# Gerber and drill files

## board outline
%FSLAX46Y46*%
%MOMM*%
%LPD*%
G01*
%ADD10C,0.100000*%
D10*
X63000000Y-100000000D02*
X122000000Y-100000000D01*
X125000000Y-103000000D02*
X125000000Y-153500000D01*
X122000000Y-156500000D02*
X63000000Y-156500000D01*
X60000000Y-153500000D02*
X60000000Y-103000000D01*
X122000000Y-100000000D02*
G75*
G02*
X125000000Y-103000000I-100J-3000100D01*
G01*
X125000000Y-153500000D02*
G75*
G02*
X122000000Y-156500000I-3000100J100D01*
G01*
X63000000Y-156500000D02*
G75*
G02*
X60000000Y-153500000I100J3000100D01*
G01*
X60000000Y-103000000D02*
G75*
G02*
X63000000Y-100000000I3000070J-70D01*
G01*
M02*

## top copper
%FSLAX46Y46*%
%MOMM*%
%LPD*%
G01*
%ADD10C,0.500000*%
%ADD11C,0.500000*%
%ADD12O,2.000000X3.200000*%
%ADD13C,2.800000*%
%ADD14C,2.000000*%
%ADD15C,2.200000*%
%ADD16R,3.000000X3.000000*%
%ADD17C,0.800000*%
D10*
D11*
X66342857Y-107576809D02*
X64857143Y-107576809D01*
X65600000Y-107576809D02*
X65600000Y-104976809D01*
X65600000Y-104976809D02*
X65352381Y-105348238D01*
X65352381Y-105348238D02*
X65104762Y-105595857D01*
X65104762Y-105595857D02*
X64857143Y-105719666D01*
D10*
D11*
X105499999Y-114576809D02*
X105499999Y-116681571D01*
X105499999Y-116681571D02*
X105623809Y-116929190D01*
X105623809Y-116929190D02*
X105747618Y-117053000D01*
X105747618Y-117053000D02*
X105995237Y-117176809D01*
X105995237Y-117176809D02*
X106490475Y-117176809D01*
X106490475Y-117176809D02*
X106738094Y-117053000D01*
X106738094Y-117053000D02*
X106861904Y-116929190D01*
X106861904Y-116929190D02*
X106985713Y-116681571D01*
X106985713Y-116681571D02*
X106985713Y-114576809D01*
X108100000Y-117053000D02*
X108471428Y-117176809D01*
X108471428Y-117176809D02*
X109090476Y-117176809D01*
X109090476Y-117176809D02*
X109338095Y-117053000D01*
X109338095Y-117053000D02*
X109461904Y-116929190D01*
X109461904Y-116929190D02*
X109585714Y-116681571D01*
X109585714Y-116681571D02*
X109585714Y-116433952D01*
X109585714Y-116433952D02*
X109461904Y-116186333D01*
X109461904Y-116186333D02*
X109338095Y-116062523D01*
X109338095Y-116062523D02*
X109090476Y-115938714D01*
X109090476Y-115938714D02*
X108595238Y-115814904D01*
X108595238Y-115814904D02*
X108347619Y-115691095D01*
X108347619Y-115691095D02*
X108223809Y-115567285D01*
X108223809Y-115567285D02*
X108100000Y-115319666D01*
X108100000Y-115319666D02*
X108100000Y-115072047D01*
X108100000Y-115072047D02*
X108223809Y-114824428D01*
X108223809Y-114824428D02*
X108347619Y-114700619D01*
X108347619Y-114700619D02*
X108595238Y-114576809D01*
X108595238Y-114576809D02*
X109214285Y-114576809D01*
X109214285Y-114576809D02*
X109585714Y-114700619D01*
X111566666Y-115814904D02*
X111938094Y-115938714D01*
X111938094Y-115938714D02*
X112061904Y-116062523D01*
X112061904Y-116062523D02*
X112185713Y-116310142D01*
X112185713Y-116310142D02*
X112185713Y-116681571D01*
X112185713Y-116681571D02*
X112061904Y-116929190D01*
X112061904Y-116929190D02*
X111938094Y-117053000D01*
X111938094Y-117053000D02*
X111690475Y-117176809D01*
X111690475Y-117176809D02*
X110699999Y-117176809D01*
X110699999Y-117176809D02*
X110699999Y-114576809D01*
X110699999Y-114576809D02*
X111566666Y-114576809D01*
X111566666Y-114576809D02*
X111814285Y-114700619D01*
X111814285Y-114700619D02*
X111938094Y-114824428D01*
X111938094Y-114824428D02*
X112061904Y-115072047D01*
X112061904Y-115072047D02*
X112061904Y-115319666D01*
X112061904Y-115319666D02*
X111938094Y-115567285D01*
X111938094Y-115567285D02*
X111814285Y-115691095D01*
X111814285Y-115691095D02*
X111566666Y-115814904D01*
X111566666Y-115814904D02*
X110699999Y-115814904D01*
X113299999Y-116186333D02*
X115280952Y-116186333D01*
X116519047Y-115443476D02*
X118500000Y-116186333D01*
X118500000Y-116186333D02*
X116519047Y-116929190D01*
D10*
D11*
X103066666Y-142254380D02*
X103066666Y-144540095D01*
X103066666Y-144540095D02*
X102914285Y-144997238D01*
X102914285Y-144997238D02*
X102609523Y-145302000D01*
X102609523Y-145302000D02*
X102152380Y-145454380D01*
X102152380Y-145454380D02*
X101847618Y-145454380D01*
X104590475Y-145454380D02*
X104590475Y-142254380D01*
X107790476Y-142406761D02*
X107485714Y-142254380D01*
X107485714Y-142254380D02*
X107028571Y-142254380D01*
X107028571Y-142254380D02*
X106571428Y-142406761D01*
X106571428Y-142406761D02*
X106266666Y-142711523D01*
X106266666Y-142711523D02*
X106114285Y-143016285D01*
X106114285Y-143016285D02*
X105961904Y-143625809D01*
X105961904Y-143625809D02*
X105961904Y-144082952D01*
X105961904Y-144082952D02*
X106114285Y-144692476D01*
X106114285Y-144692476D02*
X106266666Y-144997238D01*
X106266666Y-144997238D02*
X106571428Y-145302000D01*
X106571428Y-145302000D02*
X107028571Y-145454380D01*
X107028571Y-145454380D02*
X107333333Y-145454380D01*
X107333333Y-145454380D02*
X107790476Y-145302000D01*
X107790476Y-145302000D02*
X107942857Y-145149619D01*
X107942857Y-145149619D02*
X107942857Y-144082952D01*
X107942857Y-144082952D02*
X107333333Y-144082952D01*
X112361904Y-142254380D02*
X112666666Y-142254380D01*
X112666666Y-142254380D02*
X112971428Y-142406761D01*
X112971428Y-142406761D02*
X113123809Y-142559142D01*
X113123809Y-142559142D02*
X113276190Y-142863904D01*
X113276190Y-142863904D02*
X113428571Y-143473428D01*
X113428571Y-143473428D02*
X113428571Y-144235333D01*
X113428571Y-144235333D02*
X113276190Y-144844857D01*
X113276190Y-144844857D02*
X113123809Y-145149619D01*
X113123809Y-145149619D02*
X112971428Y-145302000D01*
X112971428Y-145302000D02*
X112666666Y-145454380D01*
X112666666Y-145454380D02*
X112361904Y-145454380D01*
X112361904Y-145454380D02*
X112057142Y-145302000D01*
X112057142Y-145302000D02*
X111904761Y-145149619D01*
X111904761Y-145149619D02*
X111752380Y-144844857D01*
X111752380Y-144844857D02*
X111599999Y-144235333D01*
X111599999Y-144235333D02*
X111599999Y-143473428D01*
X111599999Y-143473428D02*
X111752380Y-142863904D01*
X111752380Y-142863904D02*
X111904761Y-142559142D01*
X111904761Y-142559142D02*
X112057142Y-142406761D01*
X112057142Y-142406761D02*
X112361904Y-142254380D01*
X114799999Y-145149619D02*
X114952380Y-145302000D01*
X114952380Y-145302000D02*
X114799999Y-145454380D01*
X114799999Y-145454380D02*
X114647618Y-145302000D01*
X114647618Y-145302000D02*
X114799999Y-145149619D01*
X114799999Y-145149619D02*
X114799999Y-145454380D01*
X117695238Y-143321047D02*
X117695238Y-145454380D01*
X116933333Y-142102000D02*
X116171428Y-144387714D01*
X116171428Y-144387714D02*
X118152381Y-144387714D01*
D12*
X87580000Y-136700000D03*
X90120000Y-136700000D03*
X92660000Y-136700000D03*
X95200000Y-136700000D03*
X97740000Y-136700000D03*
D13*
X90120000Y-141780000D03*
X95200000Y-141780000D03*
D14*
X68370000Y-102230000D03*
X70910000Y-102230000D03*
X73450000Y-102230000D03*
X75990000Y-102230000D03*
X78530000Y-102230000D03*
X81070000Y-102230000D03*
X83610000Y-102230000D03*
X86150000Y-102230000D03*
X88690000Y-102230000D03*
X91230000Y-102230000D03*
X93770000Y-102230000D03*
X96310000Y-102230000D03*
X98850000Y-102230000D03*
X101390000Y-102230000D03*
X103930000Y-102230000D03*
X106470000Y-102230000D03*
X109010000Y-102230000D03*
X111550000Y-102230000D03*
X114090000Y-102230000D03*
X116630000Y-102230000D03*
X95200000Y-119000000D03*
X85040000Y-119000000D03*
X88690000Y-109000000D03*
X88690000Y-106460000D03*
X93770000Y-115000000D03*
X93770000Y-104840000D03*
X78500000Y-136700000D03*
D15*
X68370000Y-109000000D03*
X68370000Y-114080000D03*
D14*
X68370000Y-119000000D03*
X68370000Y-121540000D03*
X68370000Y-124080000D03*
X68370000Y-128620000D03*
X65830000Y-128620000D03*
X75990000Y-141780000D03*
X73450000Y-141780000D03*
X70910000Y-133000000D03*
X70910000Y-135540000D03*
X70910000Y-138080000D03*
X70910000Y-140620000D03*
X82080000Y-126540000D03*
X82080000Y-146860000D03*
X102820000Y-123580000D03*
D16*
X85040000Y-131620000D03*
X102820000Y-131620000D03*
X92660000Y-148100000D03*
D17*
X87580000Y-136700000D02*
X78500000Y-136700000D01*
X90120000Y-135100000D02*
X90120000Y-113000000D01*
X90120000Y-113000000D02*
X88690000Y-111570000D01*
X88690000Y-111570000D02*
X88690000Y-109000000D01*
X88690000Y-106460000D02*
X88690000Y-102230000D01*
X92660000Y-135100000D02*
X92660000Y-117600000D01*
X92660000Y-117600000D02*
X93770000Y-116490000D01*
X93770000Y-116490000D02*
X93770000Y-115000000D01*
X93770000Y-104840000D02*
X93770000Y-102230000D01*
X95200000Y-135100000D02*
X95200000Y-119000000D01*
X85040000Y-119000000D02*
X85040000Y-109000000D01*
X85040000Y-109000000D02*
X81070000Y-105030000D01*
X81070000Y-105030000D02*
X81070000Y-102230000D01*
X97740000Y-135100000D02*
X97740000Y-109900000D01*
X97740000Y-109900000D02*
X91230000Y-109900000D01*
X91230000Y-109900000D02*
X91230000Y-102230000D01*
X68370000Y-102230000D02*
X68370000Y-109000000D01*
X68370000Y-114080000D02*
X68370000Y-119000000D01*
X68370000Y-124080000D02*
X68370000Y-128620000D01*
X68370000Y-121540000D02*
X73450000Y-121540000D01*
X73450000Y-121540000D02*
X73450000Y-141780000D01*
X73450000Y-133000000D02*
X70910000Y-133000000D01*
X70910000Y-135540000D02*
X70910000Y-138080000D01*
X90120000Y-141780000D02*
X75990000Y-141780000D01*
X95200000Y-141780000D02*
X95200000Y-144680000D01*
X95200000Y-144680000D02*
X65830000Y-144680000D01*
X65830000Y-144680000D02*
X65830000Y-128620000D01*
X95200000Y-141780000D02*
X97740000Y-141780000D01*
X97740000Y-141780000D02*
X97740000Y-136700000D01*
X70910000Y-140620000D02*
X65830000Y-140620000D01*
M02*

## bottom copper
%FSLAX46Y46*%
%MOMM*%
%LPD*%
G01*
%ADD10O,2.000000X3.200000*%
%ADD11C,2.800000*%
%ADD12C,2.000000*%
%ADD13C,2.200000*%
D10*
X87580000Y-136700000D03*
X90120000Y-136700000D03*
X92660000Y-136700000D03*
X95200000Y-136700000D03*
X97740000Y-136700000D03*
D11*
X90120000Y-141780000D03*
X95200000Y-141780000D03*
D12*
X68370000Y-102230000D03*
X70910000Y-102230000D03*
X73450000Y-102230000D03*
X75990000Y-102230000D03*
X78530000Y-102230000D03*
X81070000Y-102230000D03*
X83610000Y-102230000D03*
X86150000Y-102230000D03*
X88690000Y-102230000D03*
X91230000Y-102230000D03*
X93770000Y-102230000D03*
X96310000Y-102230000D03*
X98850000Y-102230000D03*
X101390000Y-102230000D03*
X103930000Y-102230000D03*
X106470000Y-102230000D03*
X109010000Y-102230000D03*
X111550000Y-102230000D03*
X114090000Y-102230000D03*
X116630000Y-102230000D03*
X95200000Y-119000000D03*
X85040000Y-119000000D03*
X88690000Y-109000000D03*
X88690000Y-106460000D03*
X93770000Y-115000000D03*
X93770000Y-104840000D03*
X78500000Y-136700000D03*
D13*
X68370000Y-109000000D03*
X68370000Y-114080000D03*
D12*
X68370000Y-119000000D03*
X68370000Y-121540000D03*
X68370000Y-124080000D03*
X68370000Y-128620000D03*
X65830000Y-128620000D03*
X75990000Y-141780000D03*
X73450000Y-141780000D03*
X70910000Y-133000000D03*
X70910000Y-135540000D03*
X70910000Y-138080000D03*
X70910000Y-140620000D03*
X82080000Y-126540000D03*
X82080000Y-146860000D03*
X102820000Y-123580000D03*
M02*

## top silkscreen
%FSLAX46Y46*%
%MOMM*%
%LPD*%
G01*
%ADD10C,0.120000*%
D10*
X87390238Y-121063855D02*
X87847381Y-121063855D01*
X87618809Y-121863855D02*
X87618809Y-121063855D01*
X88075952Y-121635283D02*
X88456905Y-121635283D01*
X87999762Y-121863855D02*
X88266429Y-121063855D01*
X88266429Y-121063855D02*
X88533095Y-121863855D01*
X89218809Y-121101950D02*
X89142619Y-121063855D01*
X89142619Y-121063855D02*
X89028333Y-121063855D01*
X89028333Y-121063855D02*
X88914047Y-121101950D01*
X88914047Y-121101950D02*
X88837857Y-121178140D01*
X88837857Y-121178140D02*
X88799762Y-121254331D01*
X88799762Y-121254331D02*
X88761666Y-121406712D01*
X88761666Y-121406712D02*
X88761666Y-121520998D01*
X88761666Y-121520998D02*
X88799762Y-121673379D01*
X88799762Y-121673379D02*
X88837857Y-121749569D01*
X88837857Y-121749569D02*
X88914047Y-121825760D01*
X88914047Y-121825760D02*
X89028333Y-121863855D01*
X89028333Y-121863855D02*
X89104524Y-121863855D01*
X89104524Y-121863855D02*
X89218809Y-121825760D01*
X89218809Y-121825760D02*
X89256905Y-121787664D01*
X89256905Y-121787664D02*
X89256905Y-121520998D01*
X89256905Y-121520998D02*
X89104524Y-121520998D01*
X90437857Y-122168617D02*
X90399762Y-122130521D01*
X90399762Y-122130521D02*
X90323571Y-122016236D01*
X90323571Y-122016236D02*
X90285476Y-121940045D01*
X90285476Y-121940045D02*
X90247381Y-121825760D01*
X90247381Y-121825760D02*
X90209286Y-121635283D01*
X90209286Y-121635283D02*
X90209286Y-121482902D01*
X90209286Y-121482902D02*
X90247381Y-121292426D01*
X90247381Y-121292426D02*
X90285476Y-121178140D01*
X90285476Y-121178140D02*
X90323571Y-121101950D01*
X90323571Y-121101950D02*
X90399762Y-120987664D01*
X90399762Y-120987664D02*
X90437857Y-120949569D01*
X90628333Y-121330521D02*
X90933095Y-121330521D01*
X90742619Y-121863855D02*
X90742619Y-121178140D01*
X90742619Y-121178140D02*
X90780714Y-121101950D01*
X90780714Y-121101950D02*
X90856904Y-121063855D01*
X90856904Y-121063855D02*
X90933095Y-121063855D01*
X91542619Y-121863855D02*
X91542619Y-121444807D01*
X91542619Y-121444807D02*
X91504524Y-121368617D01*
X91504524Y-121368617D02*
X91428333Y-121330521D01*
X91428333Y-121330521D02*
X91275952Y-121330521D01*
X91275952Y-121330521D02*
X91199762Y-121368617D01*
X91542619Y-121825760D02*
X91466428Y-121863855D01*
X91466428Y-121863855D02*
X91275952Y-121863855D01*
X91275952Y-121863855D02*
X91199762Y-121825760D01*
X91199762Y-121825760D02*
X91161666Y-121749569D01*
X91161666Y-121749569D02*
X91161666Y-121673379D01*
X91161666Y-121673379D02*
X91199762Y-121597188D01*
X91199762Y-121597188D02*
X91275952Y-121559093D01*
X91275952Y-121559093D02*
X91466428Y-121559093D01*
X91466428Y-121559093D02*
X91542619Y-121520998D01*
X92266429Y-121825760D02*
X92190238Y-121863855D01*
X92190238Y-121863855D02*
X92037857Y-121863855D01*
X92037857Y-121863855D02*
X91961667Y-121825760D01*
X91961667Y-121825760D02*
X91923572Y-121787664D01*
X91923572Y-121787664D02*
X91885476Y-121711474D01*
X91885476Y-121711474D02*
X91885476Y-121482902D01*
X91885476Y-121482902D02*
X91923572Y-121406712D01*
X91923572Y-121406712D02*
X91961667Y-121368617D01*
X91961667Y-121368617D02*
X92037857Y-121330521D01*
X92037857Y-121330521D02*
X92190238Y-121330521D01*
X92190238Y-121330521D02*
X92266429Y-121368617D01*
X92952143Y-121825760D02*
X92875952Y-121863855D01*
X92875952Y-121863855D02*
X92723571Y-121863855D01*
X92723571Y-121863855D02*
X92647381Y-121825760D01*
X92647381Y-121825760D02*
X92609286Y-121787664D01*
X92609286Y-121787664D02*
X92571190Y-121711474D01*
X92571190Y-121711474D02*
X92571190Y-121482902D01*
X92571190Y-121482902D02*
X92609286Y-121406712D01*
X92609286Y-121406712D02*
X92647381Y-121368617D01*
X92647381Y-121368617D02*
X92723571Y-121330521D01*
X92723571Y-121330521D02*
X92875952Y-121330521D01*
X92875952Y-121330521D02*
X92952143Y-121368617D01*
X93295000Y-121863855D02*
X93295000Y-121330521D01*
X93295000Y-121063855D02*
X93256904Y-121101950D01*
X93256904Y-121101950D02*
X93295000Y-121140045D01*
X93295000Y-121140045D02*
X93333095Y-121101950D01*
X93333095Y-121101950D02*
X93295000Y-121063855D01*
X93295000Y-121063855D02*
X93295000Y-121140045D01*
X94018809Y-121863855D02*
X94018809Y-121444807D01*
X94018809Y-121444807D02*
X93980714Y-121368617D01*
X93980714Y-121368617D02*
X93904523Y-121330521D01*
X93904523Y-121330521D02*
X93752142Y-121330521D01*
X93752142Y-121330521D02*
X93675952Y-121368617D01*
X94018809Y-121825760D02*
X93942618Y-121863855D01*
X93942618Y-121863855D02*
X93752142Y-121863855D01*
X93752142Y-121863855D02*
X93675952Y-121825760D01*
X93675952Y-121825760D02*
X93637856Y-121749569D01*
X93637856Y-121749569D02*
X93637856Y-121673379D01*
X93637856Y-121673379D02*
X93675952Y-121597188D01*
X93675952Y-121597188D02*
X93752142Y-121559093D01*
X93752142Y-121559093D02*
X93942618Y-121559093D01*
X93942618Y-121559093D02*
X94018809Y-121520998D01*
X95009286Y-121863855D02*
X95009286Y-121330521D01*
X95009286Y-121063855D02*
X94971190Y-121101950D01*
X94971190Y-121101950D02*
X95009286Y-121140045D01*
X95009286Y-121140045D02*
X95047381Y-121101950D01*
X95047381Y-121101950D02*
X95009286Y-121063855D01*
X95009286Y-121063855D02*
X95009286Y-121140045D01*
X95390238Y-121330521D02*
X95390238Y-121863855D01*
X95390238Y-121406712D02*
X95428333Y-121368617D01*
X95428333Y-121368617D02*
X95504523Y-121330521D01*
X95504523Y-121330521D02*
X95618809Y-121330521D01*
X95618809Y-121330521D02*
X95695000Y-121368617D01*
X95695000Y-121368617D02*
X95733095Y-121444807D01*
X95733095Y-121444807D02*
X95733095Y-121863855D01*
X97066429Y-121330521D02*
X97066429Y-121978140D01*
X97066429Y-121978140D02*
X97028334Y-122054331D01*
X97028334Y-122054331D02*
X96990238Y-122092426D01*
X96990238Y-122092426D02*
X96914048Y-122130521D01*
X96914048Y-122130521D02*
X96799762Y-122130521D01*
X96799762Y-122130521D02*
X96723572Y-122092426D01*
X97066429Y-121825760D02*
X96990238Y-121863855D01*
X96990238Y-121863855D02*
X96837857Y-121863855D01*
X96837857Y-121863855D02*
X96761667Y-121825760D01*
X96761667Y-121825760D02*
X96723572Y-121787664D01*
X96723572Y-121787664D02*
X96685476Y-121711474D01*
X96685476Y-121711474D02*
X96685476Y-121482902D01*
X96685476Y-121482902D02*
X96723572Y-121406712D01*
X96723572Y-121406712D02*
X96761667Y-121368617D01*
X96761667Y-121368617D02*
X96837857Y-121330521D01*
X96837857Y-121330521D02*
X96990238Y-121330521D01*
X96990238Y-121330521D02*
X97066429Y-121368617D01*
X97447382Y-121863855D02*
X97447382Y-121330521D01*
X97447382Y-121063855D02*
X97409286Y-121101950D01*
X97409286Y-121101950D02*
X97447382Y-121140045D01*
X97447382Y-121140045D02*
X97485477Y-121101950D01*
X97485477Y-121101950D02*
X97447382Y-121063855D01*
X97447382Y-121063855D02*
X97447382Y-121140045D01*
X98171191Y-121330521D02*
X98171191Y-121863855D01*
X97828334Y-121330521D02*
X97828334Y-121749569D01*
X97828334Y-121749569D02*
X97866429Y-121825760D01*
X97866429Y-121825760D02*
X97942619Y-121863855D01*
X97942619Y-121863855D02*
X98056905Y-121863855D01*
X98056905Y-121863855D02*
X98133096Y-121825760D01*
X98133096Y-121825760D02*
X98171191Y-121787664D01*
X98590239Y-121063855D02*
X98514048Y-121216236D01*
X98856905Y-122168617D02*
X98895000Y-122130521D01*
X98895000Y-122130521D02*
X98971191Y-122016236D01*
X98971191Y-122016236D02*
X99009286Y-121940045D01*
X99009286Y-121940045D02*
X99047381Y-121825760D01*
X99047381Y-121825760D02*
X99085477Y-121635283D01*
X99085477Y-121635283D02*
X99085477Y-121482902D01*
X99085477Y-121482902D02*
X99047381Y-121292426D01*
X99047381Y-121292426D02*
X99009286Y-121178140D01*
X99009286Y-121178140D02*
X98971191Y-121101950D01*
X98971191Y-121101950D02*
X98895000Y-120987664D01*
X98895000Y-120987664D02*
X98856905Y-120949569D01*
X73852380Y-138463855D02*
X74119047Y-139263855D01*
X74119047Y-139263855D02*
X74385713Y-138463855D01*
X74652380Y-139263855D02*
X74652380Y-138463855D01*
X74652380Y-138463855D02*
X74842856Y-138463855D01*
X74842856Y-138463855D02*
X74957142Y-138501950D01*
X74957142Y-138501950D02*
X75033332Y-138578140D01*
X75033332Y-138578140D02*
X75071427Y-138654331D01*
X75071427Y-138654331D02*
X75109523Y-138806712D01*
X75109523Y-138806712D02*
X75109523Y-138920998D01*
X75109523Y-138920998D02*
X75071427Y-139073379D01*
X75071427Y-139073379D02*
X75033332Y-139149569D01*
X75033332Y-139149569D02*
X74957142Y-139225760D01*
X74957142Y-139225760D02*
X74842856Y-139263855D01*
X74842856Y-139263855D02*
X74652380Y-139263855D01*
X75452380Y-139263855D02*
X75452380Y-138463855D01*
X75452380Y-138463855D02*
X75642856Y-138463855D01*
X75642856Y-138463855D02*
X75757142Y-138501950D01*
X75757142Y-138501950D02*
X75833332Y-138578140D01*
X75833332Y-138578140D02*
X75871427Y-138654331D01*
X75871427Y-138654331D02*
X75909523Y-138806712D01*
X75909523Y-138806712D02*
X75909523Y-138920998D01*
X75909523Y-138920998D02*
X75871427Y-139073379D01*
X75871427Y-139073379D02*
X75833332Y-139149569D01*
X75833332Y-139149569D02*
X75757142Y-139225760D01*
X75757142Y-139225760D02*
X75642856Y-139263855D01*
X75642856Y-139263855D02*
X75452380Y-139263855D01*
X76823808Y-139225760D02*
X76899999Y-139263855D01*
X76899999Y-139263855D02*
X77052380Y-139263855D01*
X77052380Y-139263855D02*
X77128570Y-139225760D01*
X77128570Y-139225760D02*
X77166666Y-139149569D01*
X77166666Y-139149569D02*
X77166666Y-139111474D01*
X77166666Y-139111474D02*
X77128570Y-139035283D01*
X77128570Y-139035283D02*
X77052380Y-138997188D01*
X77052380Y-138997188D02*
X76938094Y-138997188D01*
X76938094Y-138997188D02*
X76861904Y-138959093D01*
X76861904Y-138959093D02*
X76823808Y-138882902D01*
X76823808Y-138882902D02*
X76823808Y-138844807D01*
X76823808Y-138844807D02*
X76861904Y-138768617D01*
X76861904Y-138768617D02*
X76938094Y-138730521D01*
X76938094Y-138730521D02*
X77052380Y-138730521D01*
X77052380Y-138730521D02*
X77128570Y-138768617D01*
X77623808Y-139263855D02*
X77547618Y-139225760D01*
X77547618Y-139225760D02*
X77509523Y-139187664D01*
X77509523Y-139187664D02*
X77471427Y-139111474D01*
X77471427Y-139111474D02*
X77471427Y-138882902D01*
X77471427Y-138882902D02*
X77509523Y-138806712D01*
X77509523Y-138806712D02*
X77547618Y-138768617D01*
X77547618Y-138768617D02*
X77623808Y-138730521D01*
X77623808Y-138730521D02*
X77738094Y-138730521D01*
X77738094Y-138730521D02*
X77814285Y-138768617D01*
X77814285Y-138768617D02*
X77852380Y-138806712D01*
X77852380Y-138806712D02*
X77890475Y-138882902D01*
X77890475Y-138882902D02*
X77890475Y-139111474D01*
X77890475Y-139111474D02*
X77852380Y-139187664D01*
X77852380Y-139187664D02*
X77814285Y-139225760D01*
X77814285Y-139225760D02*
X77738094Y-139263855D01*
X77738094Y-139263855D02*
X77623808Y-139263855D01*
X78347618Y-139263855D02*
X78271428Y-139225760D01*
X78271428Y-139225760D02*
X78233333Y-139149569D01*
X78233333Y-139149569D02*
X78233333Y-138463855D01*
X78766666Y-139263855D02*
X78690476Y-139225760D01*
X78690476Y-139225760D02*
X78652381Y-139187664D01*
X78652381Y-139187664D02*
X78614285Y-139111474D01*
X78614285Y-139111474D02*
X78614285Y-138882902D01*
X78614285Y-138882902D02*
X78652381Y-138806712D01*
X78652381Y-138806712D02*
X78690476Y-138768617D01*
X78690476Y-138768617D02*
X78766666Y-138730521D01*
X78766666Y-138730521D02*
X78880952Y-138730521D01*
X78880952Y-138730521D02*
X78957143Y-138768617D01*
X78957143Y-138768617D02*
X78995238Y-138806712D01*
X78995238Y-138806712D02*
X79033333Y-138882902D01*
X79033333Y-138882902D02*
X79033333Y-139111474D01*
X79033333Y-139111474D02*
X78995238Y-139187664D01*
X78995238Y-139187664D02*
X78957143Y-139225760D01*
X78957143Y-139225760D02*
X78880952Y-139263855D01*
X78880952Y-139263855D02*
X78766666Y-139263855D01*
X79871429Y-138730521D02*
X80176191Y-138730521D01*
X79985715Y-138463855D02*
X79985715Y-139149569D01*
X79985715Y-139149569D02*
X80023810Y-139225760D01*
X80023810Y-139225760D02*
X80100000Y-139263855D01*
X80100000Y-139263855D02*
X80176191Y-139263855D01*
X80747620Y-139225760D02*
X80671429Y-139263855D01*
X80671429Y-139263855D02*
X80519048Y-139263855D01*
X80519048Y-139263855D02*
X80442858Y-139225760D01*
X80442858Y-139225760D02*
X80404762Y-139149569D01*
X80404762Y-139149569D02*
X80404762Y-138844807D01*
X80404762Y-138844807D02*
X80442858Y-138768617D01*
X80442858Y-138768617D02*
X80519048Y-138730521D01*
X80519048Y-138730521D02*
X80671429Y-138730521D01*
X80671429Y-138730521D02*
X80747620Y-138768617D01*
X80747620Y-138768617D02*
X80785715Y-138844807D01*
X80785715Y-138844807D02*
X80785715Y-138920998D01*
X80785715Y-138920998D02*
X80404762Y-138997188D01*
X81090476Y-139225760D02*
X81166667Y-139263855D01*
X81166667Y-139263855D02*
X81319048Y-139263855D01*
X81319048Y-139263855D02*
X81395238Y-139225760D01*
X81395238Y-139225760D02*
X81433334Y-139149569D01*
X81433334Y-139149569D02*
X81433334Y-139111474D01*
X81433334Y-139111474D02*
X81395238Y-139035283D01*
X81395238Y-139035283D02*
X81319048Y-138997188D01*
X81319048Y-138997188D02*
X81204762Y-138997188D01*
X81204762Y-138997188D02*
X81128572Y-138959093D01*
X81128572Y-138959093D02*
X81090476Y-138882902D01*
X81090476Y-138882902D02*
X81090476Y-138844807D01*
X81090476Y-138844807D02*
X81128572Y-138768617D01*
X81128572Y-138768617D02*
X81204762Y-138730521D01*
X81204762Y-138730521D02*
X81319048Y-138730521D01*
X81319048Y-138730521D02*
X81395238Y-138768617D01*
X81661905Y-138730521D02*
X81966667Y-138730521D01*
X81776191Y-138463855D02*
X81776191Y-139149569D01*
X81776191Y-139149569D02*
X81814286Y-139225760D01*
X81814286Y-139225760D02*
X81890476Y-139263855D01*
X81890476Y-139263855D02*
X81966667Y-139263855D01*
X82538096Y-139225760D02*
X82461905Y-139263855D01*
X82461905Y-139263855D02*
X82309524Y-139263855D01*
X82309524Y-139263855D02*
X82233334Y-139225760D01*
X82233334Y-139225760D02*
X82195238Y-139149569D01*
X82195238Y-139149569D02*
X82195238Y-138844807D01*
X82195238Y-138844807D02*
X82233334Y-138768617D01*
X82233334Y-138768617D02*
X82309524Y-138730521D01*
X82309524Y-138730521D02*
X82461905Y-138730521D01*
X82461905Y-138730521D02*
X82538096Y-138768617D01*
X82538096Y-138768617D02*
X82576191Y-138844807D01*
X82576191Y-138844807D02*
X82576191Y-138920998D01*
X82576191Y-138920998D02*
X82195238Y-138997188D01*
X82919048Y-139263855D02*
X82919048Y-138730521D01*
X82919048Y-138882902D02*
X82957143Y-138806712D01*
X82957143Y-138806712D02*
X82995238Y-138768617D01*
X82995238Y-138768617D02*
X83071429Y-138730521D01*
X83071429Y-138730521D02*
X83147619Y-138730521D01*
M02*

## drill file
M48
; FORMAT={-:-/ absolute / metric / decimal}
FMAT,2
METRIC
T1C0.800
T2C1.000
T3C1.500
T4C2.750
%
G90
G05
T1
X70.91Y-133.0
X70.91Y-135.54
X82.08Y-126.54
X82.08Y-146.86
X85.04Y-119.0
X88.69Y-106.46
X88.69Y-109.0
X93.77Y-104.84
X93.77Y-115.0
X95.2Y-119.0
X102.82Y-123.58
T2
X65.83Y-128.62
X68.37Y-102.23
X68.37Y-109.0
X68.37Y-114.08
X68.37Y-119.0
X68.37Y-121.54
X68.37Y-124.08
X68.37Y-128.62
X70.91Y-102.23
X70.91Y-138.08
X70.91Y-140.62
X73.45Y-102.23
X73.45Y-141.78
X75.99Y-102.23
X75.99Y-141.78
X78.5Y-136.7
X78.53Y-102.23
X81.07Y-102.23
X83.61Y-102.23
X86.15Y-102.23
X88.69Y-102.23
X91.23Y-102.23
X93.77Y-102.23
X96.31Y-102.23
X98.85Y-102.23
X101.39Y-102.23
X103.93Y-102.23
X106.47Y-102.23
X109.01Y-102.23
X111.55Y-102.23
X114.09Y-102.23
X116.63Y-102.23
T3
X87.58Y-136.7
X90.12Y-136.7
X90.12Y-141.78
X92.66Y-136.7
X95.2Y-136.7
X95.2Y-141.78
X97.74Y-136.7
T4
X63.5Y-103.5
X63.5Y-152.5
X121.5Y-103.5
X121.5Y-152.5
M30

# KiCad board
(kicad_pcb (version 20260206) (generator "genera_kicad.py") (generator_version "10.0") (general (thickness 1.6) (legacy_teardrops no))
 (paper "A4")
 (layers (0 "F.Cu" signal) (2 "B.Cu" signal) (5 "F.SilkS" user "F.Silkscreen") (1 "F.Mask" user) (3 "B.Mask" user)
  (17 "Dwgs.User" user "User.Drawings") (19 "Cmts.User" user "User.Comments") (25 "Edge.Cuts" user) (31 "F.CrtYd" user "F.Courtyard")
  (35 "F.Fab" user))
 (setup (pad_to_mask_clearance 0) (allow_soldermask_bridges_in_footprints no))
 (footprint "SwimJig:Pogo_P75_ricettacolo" (layer "F.Cu") (at 87.58 136.7)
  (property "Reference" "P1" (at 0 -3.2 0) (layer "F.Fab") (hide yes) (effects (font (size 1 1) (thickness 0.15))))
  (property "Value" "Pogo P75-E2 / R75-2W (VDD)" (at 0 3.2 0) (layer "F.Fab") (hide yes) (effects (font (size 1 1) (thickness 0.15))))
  (pad "1" thru_hole oval (at 0 0) (size 2 3.2) (drill 1.5) (layers "F.Cu" "F.Mask") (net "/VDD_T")))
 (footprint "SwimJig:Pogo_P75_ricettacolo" (layer "F.Cu") (at 90.12 136.7)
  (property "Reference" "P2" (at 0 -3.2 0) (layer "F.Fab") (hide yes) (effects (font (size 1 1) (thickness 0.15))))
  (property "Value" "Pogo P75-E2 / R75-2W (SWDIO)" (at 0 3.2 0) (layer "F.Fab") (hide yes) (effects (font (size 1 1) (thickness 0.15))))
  (pad "1" thru_hole oval (at 0 0) (size 2 3.2) (drill 1.5) (layers "F.Cu" "F.Mask") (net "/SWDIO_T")))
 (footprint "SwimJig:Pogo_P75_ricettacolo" (layer "F.Cu") (at 92.66 136.7)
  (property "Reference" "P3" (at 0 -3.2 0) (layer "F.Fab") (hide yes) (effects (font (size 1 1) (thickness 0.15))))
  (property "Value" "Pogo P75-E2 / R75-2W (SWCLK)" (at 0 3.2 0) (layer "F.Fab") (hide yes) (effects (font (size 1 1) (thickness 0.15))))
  (pad "1" thru_hole oval (at 0 0) (size 2 3.2) (drill 1.5) (layers "F.Cu" "F.Mask") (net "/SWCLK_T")))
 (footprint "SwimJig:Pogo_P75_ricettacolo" (layer "F.Cu") (at 95.2 136.7)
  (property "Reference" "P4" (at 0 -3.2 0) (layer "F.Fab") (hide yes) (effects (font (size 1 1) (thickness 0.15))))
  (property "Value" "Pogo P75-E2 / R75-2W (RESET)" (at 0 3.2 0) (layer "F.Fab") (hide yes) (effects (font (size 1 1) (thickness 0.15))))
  (pad "1" thru_hole oval (at 0 0) (size 2 3.2) (drill 1.5) (layers "F.Cu" "F.Mask") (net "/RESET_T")))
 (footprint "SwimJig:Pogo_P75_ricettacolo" (layer "F.Cu") (at 97.74 136.7)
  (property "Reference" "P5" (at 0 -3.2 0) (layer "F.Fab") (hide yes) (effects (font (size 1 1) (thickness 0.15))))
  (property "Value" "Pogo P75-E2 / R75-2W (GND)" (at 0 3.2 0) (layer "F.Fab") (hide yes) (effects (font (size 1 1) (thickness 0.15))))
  (pad "1" thru_hole oval (at 0 0) (size 2 3.2) (drill 1.5) (layers "F.Cu" "F.Mask") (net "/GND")))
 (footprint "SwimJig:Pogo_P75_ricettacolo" (layer "F.Cu") (at 90.12 141.78)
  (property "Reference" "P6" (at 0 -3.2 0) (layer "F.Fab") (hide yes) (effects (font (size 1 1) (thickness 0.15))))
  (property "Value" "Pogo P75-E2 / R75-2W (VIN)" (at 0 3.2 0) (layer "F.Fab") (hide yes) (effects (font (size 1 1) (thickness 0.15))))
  (pad "1" thru_hole circle (at 0 0) (size 2.8 2.8) (drill 1.5) (layers "F.Cu" "F.Mask") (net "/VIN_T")))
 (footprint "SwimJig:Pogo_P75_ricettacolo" (layer "F.Cu") (at 95.2 141.78)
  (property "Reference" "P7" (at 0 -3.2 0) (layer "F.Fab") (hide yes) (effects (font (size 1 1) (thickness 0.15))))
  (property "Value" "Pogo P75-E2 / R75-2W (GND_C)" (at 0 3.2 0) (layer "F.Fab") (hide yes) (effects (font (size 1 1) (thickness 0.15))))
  (pad "1" thru_hole circle (at 0 0) (size 2.8 2.8) (drill 1.5) (layers "F.Cu" "F.Mask") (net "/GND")))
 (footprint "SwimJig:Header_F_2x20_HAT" (layer "F.Cu") (at 68.37 102.23)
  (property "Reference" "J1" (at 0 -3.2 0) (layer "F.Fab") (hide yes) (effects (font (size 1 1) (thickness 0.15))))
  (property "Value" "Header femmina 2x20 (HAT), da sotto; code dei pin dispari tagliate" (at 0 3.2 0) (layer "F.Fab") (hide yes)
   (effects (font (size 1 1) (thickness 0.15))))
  (pad "2" thru_hole circle (at 0 0) (size 2 2) (drill 1) (layers "F.Cu" "F.Mask") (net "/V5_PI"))
  (pad "4" thru_hole circle (at 2.54 0) (size 2 2) (drill 1) (layers "F.Cu" "F.Mask"))
  (pad "6" thru_hole circle (at 5.08 0) (size 2 2) (drill 1) (layers "F.Cu" "F.Mask"))
  (pad "8" thru_hole circle (at 7.62 0) (size 2 2) (drill 1) (layers "F.Cu" "F.Mask"))
  (pad "10" thru_hole circle (at 10.16 0) (size 2 2) (drill 1) (layers "F.Cu" "F.Mask"))
  (pad "12" thru_hole circle (at 12.7 0) (size 2 2) (drill 1) (layers "F.Cu" "F.Mask") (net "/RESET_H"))
  (pad "14" thru_hole circle (at 15.24 0) (size 2 2) (drill 1) (layers "F.Cu" "F.Mask"))
  (pad "16" thru_hole circle (at 17.78 0) (size 2 2) (drill 1) (layers "F.Cu" "F.Mask"))
  (pad "18" thru_hole circle (at 20.32 0) (size 2 2) (drill 1) (layers "F.Cu" "F.Mask") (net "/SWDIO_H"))
  (pad "20" thru_hole circle (at 22.86 0) (size 2 2) (drill 1) (layers "F.Cu" "F.Mask") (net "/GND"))
  (pad "22" thru_hole circle (at 25.4 0) (size 2 2) (drill 1) (layers "F.Cu" "F.Mask") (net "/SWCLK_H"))
  (pad "24" thru_hole circle (at 27.94 0) (size 2 2) (drill 1) (layers "F.Cu" "F.Mask"))
  (pad "26" thru_hole circle (at 30.48 0) (size 2 2) (drill 1) (layers "F.Cu" "F.Mask"))
  (pad "28" thru_hole circle (at 33.02 0) (size 2 2) (drill 1) (layers "F.Cu" "F.Mask"))
  (pad "30" thru_hole circle (at 35.56 0) (size 2 2) (drill 1) (layers "F.Cu" "F.Mask"))
  (pad "32" thru_hole circle (at 38.1 0) (size 2 2) (drill 1) (layers "F.Cu" "F.Mask"))
  (pad "34" thru_hole circle (at 40.64 0) (size 2 2) (drill 1) (layers "F.Cu" "F.Mask"))
  (pad "36" thru_hole circle (at 43.18 0) (size 2 2) (drill 1) (layers "F.Cu" "F.Mask"))
  (pad "38" thru_hole circle (at 45.72 0) (size 2 2) (drill 1) (layers "F.Cu" "F.Mask"))
  (pad "40" thru_hole circle (at 48.26 0) (size 2 2) (drill 1) (layers "F.Cu" "F.Mask")))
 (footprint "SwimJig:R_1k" (layer "F.Cu") (at 95.2 119)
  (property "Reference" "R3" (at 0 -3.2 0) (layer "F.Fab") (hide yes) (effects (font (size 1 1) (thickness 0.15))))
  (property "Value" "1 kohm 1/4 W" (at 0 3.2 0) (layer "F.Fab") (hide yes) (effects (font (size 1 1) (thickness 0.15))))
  (pad "1" thru_hole circle (at 0 0) (size 2 2) (drill 0.8) (layers "F.Cu" "F.Mask") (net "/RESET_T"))
  (pad "2" thru_hole circle (at -10.16 0) (size 2 2) (drill 0.8) (layers "F.Cu" "F.Mask") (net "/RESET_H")))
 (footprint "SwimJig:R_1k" (layer "F.Cu") (at 88.69 109)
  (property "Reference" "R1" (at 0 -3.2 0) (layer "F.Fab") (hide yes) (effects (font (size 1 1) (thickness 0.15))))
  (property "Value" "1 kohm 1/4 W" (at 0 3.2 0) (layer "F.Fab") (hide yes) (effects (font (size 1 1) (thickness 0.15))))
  (pad "1" thru_hole circle (at 0 0) (size 2 2) (drill 0.8) (layers "F.Cu" "F.Mask") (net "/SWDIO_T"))
  (pad "2" thru_hole circle (at 0 -2.54) (size 2 2) (drill 0.8) (layers "F.Cu" "F.Mask") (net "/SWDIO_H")))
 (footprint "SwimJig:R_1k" (layer "F.Cu") (at 93.77 115)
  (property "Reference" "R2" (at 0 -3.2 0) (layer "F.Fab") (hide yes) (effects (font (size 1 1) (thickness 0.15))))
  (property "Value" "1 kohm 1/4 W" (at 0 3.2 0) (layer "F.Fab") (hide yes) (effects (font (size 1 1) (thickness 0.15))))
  (pad "1" thru_hole circle (at 0 0) (size 2 2) (drill 0.8) (layers "F.Cu" "F.Mask") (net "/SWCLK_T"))
  (pad "2" thru_hole circle (at 0 -10.16) (size 2 2) (drill 0.8) (layers "F.Cu" "F.Mask") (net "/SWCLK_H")))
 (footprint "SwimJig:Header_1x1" (layer "F.Cu") (at 78.5 136.7)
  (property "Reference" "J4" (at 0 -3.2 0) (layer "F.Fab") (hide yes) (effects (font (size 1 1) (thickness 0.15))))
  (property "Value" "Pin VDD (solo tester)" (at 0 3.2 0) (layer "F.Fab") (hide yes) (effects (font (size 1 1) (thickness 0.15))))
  (pad "1" thru_hole circle (at 0 0) (size 2 2) (drill 1) (layers "F.Cu" "F.Mask") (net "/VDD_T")))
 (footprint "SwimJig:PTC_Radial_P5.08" (layer "F.Cu") (at 68.37 109)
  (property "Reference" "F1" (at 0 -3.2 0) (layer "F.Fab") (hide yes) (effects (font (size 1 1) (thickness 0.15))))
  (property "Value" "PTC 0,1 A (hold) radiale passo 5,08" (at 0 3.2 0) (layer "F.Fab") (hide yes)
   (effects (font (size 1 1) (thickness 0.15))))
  (pad "1" thru_hole circle (at 0 0) (size 2.2 2.2) (drill 1) (layers "F.Cu" "F.Mask") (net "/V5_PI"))
  (pad "2" thru_hole circle (at 0 5.08) (size 2.2 2.2) (drill 1) (layers "F.Cu" "F.Mask") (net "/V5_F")))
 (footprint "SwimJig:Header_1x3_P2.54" (layer "F.Cu") (at 68.37 119)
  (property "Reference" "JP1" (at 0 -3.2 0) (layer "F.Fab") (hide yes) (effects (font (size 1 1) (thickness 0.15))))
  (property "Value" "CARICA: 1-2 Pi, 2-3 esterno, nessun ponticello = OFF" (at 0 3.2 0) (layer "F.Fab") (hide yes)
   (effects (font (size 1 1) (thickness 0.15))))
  (pad "1" thru_hole circle (at 0 0) (size 2 2) (drill 1) (layers "F.Cu" "F.Mask") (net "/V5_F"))
  (pad "2" thru_hole circle (at 0 2.54) (size 2 2) (drill 1) (layers "F.Cu" "F.Mask") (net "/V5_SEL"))
  (pad "3" thru_hole circle (at 0 5.08) (size 2 2) (drill 1) (layers "F.Cu" "F.Mask") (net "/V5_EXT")))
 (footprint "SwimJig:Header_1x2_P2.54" (layer "F.Cu") (at 68.37 128.62)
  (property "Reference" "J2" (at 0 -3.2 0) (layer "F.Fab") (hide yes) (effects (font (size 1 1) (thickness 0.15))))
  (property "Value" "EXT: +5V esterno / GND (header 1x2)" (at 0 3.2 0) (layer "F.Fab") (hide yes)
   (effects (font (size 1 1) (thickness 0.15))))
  (pad "1" thru_hole circle (at 0 0) (size 2 2) (drill 1) (layers "F.Cu" "F.Mask") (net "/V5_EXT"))
  (pad "2" thru_hole circle (at -2.54 0) (size 2 2) (drill 1) (layers "F.Cu" "F.Mask") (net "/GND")))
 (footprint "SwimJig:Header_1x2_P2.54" (layer "F.Cu") (at 75.99 141.78)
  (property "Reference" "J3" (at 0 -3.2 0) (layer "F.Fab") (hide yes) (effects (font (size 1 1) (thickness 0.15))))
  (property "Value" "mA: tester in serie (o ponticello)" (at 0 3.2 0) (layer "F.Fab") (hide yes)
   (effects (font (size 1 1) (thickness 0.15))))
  (pad "1" thru_hole circle (at 0 0) (size 2 2) (drill 1) (layers "F.Cu" "F.Mask") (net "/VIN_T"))
  (pad "2" thru_hole circle (at -2.54 0) (size 2 2) (drill 1) (layers "F.Cu" "F.Mask") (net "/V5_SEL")))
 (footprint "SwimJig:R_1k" (layer "F.Cu") (at 70.91 133)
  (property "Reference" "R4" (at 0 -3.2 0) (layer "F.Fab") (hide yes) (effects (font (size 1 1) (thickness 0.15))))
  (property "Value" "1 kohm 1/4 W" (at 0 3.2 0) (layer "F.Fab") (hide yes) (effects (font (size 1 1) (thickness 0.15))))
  (pad "1" thru_hole circle (at 0 0) (size 2 2) (drill 0.8) (layers "F.Cu" "F.Mask") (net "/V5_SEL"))
  (pad "2" thru_hole circle (at 0 2.54) (size 2 2) (drill 0.8) (layers "F.Cu" "F.Mask") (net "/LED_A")))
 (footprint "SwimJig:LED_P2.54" (layer "F.Cu") (at 70.91 138.08)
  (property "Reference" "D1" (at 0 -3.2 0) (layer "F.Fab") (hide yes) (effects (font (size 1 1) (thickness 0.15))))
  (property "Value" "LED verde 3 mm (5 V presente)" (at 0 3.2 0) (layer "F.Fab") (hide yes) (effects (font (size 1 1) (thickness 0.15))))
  (pad "1" thru_hole circle (at 0 0) (size 2 2) (drill 1) (layers "F.Cu" "F.Mask") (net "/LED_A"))
  (pad "2" thru_hole circle (at 0 2.54) (size 2 2) (drill 1) (layers "F.Cu" "F.Mask") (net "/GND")))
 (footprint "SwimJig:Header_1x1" (layer "F.Cu") (at 82.08 126.54)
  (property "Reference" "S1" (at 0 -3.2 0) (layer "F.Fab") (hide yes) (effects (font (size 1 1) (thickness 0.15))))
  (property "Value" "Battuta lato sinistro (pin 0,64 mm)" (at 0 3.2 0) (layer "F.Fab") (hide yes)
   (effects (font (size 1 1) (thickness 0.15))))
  (pad "1" thru_hole circle (at 0 0) (size 2 2) (drill 0.8) (layers "F.Cu" "F.Mask")))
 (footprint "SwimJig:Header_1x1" (layer "F.Cu") (at 82.08 146.86)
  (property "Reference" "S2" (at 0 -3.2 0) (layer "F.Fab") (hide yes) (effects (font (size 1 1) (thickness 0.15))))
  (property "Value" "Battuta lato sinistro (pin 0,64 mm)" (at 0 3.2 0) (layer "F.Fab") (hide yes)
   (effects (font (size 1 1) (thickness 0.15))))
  (pad "1" thru_hole circle (at 0 0) (size 2 2) (drill 0.8) (layers "F.Cu" "F.Mask")))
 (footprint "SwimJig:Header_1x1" (layer "F.Cu") (at 102.82 123.58)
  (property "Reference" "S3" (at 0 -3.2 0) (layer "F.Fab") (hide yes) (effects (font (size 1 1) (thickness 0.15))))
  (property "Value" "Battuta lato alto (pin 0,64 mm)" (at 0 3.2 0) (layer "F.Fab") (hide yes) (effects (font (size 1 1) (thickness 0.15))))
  (pad "1" thru_hole circle (at 0 0) (size 2 2) (drill 0.8) (layers "F.Cu" "F.Mask")))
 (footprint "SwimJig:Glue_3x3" (layer "F.Cu") (at 85.04 131.62)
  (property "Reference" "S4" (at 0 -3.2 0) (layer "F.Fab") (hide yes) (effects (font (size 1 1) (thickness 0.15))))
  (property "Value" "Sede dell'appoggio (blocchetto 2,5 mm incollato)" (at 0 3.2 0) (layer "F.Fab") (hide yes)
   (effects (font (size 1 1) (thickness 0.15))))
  (pad "1" smd rect (at 0 0) (size 3 3) (layers "F.Cu" "F.Mask")))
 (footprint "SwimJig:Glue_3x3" (layer "F.Cu") (at 102.82 131.62)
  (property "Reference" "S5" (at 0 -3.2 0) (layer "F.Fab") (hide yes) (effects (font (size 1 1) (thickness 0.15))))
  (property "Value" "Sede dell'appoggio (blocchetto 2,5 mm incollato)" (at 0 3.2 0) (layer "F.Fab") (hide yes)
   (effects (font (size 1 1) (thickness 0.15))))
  (pad "1" smd rect (at 0 0) (size 3 3) (layers "F.Cu" "F.Mask")))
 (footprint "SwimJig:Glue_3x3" (layer "F.Cu") (at 92.66 148.1)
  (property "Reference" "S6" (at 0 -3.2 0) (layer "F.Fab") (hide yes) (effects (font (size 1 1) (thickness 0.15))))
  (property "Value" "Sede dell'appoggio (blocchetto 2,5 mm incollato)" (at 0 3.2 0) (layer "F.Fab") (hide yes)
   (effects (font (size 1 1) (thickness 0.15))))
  (pad "1" smd rect (at 0 0) (size 3 3) (layers "F.Cu" "F.Mask")))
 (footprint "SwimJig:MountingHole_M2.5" (layer "F.Cu") (at 63.5 103.5)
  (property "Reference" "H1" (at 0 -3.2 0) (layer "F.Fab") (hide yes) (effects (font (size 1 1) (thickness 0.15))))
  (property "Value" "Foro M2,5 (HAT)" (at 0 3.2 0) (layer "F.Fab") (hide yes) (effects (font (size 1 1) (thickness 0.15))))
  (pad "" np_thru_hole circle (at 0 0) (size 2.75 2.75) (drill 2.75) (layers "*.Cu" "*.Mask")))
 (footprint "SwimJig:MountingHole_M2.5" (layer "F.Cu") (at 121.5 103.5)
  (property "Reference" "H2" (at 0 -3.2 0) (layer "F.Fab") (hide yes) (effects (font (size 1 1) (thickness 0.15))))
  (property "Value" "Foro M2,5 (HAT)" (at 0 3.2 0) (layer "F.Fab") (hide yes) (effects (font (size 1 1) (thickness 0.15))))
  (pad "" np_thru_hole circle (at 0 0) (size 2.75 2.75) (drill 2.75) (layers "*.Cu" "*.Mask")))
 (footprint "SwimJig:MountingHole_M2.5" (layer "F.Cu") (at 63.5 152.5)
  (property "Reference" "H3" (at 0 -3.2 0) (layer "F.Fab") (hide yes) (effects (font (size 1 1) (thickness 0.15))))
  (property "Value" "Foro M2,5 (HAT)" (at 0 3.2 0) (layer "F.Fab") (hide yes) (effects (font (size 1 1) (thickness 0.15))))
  (pad "" np_thru_hole circle (at 0 0) (size 2.75 2.75) (drill 2.75) (layers "*.Cu" "*.Mask")))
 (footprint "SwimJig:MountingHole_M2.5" (layer "F.Cu") (at 121.5 152.5)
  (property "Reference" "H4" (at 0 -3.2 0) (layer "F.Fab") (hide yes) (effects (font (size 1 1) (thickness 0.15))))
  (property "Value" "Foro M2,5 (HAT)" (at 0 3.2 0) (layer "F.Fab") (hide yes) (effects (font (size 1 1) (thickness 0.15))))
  (pad "" np_thru_hole circle (at 0 0) (size 2.75 2.75) (drill 2.75) (layers "*.Cu" "*.Mask")))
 (segment (start 87.58 136.7) (end 78.5 136.7) (width 0.8) (layer "F.Cu") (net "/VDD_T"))
 (segment (start 90.12 135.1) (end 90.12 113) (width 0.8) (layer "F.Cu") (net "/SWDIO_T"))
 (segment (start 90.12 113) (end 88.69 111.57) (width 0.8) (layer "F.Cu") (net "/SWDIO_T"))
 (segment (start 88.69 111.57) (end 88.69 109) (width 0.8) (layer "F.Cu") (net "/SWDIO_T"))
 (segment (start 88.69 106.46) (end 88.69 102.23) (width 0.8) (layer "F.Cu") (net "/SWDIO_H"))
 (segment (start 92.66 135.1) (end 92.66 117.6) (width 0.8) (layer "F.Cu") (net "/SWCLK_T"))
 (segment (start 92.66 117.6) (end 93.77 116.49) (width 0.8) (layer "F.Cu") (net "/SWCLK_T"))
 (segment (start 93.77 116.49) (end 93.77 115) (width 0.8) (layer "F.Cu") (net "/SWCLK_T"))
 (segment (start 93.77 104.84) (end 93.77 102.23) (width 0.8) (layer "F.Cu") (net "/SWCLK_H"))
 (segment (start 95.2 135.1) (end 95.2 119) (width 0.8) (layer "F.Cu") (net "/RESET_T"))
 (segment (start 85.04 119) (end 85.04 109) (width 0.8) (layer "F.Cu") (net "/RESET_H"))
 (segment (start 85.04 109) (end 81.07 105.03) (width 0.8) (layer "F.Cu") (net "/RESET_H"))
 (segment (start 81.07 105.03) (end 81.07 102.23) (width 0.8) (layer "F.Cu") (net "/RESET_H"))
 (segment (start 97.74 135.1) (end 97.74 109.9) (width 0.8) (layer "F.Cu") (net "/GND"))
 (segment (start 97.74 109.9) (end 91.23 109.9) (width 0.8) (layer "F.Cu") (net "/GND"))
 (segment (start 91.23 109.9) (end 91.23 102.23) (width 0.8) (layer "F.Cu") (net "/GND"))
 (segment (start 68.37 102.23) (end 68.37 109) (width 0.8) (layer "F.Cu") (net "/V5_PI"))
 (segment (start 68.37 114.08) (end 68.37 119) (width 0.8) (layer "F.Cu") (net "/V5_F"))
 (segment (start 68.37 124.08) (end 68.37 128.62) (width 0.8) (layer "F.Cu") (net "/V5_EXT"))
 (segment (start 68.37 121.54) (end 73.45 121.54) (width 0.8) (layer "F.Cu") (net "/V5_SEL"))
 (segment (start 73.45 121.54) (end 73.45 141.78) (width 0.8) (layer "F.Cu") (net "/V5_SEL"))
 (segment (start 73.45 133) (end 70.91 133) (width 0.8) (layer "F.Cu") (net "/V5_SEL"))
 (segment (start 70.91 135.54) (end 70.91 138.08) (width 0.8) (layer "F.Cu") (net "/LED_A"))
 (segment (start 90.12 141.78) (end 75.99 141.78) (width 0.8) (layer "F.Cu") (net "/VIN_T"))
 (segment (start 95.2 141.78) (end 95.2 144.68) (width 0.8) (layer "F.Cu") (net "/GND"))
 (segment (start 95.2 144.68) (end 65.83 144.68) (width 0.8) (layer "F.Cu") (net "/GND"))
 (segment (start 65.83 144.68) (end 65.83 128.62) (width 0.8) (layer "F.Cu") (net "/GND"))
 (segment (start 95.2 141.78) (end 97.74 141.78) (width 0.8) (layer "F.Cu") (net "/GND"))
 (segment (start 97.74 141.78) (end 97.74 136.7) (width 0.8) (layer "F.Cu") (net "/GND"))
 (segment (start 70.91 140.62) (end 65.83 140.62) (width 0.8) (layer "F.Cu") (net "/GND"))
 (gr_line (start 63 100) (end 122 100) (stroke (width 0.1) (type default)) (layer "Edge.Cuts"))
 (gr_line (start 125 103) (end 125 153.5) (stroke (width 0.1) (type default)) (layer "Edge.Cuts"))
 (gr_line (start 122 156.5) (end 63 156.5) (stroke (width 0.1) (type default)) (layer "Edge.Cuts"))
 (gr_line (start 60 153.5) (end 60 103) (stroke (width 0.1) (type default)) (layer "Edge.Cuts"))
 (gr_arc (start 122 100) (mid 124.1213 100.8787) (end 125 103) (stroke (width 0.1) (type default)) (layer "Edge.Cuts"))
 (gr_arc (start 125 153.5) (mid 124.1213 155.6213) (end 122 156.5) (stroke (width 0.1) (type default)) (layer "Edge.Cuts"))
 (gr_arc (start 63 156.5) (mid 60.8787 155.6213) (end 60 153.5) (stroke (width 0.1) (type default)) (layer "Edge.Cuts"))
 (gr_arc (start 60 103) (mid 60.8787 100.8787) (end 63 100) (stroke (width 0.1) (type default)) (layer "Edge.Cuts"))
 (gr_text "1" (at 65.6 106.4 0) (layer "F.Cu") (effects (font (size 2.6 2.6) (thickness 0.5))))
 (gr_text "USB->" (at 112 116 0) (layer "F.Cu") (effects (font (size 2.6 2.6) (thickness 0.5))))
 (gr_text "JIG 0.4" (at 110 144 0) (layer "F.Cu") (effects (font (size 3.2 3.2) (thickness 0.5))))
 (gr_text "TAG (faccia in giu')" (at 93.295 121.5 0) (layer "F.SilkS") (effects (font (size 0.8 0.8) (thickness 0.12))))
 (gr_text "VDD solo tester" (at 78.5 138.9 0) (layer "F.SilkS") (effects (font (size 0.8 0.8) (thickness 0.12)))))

